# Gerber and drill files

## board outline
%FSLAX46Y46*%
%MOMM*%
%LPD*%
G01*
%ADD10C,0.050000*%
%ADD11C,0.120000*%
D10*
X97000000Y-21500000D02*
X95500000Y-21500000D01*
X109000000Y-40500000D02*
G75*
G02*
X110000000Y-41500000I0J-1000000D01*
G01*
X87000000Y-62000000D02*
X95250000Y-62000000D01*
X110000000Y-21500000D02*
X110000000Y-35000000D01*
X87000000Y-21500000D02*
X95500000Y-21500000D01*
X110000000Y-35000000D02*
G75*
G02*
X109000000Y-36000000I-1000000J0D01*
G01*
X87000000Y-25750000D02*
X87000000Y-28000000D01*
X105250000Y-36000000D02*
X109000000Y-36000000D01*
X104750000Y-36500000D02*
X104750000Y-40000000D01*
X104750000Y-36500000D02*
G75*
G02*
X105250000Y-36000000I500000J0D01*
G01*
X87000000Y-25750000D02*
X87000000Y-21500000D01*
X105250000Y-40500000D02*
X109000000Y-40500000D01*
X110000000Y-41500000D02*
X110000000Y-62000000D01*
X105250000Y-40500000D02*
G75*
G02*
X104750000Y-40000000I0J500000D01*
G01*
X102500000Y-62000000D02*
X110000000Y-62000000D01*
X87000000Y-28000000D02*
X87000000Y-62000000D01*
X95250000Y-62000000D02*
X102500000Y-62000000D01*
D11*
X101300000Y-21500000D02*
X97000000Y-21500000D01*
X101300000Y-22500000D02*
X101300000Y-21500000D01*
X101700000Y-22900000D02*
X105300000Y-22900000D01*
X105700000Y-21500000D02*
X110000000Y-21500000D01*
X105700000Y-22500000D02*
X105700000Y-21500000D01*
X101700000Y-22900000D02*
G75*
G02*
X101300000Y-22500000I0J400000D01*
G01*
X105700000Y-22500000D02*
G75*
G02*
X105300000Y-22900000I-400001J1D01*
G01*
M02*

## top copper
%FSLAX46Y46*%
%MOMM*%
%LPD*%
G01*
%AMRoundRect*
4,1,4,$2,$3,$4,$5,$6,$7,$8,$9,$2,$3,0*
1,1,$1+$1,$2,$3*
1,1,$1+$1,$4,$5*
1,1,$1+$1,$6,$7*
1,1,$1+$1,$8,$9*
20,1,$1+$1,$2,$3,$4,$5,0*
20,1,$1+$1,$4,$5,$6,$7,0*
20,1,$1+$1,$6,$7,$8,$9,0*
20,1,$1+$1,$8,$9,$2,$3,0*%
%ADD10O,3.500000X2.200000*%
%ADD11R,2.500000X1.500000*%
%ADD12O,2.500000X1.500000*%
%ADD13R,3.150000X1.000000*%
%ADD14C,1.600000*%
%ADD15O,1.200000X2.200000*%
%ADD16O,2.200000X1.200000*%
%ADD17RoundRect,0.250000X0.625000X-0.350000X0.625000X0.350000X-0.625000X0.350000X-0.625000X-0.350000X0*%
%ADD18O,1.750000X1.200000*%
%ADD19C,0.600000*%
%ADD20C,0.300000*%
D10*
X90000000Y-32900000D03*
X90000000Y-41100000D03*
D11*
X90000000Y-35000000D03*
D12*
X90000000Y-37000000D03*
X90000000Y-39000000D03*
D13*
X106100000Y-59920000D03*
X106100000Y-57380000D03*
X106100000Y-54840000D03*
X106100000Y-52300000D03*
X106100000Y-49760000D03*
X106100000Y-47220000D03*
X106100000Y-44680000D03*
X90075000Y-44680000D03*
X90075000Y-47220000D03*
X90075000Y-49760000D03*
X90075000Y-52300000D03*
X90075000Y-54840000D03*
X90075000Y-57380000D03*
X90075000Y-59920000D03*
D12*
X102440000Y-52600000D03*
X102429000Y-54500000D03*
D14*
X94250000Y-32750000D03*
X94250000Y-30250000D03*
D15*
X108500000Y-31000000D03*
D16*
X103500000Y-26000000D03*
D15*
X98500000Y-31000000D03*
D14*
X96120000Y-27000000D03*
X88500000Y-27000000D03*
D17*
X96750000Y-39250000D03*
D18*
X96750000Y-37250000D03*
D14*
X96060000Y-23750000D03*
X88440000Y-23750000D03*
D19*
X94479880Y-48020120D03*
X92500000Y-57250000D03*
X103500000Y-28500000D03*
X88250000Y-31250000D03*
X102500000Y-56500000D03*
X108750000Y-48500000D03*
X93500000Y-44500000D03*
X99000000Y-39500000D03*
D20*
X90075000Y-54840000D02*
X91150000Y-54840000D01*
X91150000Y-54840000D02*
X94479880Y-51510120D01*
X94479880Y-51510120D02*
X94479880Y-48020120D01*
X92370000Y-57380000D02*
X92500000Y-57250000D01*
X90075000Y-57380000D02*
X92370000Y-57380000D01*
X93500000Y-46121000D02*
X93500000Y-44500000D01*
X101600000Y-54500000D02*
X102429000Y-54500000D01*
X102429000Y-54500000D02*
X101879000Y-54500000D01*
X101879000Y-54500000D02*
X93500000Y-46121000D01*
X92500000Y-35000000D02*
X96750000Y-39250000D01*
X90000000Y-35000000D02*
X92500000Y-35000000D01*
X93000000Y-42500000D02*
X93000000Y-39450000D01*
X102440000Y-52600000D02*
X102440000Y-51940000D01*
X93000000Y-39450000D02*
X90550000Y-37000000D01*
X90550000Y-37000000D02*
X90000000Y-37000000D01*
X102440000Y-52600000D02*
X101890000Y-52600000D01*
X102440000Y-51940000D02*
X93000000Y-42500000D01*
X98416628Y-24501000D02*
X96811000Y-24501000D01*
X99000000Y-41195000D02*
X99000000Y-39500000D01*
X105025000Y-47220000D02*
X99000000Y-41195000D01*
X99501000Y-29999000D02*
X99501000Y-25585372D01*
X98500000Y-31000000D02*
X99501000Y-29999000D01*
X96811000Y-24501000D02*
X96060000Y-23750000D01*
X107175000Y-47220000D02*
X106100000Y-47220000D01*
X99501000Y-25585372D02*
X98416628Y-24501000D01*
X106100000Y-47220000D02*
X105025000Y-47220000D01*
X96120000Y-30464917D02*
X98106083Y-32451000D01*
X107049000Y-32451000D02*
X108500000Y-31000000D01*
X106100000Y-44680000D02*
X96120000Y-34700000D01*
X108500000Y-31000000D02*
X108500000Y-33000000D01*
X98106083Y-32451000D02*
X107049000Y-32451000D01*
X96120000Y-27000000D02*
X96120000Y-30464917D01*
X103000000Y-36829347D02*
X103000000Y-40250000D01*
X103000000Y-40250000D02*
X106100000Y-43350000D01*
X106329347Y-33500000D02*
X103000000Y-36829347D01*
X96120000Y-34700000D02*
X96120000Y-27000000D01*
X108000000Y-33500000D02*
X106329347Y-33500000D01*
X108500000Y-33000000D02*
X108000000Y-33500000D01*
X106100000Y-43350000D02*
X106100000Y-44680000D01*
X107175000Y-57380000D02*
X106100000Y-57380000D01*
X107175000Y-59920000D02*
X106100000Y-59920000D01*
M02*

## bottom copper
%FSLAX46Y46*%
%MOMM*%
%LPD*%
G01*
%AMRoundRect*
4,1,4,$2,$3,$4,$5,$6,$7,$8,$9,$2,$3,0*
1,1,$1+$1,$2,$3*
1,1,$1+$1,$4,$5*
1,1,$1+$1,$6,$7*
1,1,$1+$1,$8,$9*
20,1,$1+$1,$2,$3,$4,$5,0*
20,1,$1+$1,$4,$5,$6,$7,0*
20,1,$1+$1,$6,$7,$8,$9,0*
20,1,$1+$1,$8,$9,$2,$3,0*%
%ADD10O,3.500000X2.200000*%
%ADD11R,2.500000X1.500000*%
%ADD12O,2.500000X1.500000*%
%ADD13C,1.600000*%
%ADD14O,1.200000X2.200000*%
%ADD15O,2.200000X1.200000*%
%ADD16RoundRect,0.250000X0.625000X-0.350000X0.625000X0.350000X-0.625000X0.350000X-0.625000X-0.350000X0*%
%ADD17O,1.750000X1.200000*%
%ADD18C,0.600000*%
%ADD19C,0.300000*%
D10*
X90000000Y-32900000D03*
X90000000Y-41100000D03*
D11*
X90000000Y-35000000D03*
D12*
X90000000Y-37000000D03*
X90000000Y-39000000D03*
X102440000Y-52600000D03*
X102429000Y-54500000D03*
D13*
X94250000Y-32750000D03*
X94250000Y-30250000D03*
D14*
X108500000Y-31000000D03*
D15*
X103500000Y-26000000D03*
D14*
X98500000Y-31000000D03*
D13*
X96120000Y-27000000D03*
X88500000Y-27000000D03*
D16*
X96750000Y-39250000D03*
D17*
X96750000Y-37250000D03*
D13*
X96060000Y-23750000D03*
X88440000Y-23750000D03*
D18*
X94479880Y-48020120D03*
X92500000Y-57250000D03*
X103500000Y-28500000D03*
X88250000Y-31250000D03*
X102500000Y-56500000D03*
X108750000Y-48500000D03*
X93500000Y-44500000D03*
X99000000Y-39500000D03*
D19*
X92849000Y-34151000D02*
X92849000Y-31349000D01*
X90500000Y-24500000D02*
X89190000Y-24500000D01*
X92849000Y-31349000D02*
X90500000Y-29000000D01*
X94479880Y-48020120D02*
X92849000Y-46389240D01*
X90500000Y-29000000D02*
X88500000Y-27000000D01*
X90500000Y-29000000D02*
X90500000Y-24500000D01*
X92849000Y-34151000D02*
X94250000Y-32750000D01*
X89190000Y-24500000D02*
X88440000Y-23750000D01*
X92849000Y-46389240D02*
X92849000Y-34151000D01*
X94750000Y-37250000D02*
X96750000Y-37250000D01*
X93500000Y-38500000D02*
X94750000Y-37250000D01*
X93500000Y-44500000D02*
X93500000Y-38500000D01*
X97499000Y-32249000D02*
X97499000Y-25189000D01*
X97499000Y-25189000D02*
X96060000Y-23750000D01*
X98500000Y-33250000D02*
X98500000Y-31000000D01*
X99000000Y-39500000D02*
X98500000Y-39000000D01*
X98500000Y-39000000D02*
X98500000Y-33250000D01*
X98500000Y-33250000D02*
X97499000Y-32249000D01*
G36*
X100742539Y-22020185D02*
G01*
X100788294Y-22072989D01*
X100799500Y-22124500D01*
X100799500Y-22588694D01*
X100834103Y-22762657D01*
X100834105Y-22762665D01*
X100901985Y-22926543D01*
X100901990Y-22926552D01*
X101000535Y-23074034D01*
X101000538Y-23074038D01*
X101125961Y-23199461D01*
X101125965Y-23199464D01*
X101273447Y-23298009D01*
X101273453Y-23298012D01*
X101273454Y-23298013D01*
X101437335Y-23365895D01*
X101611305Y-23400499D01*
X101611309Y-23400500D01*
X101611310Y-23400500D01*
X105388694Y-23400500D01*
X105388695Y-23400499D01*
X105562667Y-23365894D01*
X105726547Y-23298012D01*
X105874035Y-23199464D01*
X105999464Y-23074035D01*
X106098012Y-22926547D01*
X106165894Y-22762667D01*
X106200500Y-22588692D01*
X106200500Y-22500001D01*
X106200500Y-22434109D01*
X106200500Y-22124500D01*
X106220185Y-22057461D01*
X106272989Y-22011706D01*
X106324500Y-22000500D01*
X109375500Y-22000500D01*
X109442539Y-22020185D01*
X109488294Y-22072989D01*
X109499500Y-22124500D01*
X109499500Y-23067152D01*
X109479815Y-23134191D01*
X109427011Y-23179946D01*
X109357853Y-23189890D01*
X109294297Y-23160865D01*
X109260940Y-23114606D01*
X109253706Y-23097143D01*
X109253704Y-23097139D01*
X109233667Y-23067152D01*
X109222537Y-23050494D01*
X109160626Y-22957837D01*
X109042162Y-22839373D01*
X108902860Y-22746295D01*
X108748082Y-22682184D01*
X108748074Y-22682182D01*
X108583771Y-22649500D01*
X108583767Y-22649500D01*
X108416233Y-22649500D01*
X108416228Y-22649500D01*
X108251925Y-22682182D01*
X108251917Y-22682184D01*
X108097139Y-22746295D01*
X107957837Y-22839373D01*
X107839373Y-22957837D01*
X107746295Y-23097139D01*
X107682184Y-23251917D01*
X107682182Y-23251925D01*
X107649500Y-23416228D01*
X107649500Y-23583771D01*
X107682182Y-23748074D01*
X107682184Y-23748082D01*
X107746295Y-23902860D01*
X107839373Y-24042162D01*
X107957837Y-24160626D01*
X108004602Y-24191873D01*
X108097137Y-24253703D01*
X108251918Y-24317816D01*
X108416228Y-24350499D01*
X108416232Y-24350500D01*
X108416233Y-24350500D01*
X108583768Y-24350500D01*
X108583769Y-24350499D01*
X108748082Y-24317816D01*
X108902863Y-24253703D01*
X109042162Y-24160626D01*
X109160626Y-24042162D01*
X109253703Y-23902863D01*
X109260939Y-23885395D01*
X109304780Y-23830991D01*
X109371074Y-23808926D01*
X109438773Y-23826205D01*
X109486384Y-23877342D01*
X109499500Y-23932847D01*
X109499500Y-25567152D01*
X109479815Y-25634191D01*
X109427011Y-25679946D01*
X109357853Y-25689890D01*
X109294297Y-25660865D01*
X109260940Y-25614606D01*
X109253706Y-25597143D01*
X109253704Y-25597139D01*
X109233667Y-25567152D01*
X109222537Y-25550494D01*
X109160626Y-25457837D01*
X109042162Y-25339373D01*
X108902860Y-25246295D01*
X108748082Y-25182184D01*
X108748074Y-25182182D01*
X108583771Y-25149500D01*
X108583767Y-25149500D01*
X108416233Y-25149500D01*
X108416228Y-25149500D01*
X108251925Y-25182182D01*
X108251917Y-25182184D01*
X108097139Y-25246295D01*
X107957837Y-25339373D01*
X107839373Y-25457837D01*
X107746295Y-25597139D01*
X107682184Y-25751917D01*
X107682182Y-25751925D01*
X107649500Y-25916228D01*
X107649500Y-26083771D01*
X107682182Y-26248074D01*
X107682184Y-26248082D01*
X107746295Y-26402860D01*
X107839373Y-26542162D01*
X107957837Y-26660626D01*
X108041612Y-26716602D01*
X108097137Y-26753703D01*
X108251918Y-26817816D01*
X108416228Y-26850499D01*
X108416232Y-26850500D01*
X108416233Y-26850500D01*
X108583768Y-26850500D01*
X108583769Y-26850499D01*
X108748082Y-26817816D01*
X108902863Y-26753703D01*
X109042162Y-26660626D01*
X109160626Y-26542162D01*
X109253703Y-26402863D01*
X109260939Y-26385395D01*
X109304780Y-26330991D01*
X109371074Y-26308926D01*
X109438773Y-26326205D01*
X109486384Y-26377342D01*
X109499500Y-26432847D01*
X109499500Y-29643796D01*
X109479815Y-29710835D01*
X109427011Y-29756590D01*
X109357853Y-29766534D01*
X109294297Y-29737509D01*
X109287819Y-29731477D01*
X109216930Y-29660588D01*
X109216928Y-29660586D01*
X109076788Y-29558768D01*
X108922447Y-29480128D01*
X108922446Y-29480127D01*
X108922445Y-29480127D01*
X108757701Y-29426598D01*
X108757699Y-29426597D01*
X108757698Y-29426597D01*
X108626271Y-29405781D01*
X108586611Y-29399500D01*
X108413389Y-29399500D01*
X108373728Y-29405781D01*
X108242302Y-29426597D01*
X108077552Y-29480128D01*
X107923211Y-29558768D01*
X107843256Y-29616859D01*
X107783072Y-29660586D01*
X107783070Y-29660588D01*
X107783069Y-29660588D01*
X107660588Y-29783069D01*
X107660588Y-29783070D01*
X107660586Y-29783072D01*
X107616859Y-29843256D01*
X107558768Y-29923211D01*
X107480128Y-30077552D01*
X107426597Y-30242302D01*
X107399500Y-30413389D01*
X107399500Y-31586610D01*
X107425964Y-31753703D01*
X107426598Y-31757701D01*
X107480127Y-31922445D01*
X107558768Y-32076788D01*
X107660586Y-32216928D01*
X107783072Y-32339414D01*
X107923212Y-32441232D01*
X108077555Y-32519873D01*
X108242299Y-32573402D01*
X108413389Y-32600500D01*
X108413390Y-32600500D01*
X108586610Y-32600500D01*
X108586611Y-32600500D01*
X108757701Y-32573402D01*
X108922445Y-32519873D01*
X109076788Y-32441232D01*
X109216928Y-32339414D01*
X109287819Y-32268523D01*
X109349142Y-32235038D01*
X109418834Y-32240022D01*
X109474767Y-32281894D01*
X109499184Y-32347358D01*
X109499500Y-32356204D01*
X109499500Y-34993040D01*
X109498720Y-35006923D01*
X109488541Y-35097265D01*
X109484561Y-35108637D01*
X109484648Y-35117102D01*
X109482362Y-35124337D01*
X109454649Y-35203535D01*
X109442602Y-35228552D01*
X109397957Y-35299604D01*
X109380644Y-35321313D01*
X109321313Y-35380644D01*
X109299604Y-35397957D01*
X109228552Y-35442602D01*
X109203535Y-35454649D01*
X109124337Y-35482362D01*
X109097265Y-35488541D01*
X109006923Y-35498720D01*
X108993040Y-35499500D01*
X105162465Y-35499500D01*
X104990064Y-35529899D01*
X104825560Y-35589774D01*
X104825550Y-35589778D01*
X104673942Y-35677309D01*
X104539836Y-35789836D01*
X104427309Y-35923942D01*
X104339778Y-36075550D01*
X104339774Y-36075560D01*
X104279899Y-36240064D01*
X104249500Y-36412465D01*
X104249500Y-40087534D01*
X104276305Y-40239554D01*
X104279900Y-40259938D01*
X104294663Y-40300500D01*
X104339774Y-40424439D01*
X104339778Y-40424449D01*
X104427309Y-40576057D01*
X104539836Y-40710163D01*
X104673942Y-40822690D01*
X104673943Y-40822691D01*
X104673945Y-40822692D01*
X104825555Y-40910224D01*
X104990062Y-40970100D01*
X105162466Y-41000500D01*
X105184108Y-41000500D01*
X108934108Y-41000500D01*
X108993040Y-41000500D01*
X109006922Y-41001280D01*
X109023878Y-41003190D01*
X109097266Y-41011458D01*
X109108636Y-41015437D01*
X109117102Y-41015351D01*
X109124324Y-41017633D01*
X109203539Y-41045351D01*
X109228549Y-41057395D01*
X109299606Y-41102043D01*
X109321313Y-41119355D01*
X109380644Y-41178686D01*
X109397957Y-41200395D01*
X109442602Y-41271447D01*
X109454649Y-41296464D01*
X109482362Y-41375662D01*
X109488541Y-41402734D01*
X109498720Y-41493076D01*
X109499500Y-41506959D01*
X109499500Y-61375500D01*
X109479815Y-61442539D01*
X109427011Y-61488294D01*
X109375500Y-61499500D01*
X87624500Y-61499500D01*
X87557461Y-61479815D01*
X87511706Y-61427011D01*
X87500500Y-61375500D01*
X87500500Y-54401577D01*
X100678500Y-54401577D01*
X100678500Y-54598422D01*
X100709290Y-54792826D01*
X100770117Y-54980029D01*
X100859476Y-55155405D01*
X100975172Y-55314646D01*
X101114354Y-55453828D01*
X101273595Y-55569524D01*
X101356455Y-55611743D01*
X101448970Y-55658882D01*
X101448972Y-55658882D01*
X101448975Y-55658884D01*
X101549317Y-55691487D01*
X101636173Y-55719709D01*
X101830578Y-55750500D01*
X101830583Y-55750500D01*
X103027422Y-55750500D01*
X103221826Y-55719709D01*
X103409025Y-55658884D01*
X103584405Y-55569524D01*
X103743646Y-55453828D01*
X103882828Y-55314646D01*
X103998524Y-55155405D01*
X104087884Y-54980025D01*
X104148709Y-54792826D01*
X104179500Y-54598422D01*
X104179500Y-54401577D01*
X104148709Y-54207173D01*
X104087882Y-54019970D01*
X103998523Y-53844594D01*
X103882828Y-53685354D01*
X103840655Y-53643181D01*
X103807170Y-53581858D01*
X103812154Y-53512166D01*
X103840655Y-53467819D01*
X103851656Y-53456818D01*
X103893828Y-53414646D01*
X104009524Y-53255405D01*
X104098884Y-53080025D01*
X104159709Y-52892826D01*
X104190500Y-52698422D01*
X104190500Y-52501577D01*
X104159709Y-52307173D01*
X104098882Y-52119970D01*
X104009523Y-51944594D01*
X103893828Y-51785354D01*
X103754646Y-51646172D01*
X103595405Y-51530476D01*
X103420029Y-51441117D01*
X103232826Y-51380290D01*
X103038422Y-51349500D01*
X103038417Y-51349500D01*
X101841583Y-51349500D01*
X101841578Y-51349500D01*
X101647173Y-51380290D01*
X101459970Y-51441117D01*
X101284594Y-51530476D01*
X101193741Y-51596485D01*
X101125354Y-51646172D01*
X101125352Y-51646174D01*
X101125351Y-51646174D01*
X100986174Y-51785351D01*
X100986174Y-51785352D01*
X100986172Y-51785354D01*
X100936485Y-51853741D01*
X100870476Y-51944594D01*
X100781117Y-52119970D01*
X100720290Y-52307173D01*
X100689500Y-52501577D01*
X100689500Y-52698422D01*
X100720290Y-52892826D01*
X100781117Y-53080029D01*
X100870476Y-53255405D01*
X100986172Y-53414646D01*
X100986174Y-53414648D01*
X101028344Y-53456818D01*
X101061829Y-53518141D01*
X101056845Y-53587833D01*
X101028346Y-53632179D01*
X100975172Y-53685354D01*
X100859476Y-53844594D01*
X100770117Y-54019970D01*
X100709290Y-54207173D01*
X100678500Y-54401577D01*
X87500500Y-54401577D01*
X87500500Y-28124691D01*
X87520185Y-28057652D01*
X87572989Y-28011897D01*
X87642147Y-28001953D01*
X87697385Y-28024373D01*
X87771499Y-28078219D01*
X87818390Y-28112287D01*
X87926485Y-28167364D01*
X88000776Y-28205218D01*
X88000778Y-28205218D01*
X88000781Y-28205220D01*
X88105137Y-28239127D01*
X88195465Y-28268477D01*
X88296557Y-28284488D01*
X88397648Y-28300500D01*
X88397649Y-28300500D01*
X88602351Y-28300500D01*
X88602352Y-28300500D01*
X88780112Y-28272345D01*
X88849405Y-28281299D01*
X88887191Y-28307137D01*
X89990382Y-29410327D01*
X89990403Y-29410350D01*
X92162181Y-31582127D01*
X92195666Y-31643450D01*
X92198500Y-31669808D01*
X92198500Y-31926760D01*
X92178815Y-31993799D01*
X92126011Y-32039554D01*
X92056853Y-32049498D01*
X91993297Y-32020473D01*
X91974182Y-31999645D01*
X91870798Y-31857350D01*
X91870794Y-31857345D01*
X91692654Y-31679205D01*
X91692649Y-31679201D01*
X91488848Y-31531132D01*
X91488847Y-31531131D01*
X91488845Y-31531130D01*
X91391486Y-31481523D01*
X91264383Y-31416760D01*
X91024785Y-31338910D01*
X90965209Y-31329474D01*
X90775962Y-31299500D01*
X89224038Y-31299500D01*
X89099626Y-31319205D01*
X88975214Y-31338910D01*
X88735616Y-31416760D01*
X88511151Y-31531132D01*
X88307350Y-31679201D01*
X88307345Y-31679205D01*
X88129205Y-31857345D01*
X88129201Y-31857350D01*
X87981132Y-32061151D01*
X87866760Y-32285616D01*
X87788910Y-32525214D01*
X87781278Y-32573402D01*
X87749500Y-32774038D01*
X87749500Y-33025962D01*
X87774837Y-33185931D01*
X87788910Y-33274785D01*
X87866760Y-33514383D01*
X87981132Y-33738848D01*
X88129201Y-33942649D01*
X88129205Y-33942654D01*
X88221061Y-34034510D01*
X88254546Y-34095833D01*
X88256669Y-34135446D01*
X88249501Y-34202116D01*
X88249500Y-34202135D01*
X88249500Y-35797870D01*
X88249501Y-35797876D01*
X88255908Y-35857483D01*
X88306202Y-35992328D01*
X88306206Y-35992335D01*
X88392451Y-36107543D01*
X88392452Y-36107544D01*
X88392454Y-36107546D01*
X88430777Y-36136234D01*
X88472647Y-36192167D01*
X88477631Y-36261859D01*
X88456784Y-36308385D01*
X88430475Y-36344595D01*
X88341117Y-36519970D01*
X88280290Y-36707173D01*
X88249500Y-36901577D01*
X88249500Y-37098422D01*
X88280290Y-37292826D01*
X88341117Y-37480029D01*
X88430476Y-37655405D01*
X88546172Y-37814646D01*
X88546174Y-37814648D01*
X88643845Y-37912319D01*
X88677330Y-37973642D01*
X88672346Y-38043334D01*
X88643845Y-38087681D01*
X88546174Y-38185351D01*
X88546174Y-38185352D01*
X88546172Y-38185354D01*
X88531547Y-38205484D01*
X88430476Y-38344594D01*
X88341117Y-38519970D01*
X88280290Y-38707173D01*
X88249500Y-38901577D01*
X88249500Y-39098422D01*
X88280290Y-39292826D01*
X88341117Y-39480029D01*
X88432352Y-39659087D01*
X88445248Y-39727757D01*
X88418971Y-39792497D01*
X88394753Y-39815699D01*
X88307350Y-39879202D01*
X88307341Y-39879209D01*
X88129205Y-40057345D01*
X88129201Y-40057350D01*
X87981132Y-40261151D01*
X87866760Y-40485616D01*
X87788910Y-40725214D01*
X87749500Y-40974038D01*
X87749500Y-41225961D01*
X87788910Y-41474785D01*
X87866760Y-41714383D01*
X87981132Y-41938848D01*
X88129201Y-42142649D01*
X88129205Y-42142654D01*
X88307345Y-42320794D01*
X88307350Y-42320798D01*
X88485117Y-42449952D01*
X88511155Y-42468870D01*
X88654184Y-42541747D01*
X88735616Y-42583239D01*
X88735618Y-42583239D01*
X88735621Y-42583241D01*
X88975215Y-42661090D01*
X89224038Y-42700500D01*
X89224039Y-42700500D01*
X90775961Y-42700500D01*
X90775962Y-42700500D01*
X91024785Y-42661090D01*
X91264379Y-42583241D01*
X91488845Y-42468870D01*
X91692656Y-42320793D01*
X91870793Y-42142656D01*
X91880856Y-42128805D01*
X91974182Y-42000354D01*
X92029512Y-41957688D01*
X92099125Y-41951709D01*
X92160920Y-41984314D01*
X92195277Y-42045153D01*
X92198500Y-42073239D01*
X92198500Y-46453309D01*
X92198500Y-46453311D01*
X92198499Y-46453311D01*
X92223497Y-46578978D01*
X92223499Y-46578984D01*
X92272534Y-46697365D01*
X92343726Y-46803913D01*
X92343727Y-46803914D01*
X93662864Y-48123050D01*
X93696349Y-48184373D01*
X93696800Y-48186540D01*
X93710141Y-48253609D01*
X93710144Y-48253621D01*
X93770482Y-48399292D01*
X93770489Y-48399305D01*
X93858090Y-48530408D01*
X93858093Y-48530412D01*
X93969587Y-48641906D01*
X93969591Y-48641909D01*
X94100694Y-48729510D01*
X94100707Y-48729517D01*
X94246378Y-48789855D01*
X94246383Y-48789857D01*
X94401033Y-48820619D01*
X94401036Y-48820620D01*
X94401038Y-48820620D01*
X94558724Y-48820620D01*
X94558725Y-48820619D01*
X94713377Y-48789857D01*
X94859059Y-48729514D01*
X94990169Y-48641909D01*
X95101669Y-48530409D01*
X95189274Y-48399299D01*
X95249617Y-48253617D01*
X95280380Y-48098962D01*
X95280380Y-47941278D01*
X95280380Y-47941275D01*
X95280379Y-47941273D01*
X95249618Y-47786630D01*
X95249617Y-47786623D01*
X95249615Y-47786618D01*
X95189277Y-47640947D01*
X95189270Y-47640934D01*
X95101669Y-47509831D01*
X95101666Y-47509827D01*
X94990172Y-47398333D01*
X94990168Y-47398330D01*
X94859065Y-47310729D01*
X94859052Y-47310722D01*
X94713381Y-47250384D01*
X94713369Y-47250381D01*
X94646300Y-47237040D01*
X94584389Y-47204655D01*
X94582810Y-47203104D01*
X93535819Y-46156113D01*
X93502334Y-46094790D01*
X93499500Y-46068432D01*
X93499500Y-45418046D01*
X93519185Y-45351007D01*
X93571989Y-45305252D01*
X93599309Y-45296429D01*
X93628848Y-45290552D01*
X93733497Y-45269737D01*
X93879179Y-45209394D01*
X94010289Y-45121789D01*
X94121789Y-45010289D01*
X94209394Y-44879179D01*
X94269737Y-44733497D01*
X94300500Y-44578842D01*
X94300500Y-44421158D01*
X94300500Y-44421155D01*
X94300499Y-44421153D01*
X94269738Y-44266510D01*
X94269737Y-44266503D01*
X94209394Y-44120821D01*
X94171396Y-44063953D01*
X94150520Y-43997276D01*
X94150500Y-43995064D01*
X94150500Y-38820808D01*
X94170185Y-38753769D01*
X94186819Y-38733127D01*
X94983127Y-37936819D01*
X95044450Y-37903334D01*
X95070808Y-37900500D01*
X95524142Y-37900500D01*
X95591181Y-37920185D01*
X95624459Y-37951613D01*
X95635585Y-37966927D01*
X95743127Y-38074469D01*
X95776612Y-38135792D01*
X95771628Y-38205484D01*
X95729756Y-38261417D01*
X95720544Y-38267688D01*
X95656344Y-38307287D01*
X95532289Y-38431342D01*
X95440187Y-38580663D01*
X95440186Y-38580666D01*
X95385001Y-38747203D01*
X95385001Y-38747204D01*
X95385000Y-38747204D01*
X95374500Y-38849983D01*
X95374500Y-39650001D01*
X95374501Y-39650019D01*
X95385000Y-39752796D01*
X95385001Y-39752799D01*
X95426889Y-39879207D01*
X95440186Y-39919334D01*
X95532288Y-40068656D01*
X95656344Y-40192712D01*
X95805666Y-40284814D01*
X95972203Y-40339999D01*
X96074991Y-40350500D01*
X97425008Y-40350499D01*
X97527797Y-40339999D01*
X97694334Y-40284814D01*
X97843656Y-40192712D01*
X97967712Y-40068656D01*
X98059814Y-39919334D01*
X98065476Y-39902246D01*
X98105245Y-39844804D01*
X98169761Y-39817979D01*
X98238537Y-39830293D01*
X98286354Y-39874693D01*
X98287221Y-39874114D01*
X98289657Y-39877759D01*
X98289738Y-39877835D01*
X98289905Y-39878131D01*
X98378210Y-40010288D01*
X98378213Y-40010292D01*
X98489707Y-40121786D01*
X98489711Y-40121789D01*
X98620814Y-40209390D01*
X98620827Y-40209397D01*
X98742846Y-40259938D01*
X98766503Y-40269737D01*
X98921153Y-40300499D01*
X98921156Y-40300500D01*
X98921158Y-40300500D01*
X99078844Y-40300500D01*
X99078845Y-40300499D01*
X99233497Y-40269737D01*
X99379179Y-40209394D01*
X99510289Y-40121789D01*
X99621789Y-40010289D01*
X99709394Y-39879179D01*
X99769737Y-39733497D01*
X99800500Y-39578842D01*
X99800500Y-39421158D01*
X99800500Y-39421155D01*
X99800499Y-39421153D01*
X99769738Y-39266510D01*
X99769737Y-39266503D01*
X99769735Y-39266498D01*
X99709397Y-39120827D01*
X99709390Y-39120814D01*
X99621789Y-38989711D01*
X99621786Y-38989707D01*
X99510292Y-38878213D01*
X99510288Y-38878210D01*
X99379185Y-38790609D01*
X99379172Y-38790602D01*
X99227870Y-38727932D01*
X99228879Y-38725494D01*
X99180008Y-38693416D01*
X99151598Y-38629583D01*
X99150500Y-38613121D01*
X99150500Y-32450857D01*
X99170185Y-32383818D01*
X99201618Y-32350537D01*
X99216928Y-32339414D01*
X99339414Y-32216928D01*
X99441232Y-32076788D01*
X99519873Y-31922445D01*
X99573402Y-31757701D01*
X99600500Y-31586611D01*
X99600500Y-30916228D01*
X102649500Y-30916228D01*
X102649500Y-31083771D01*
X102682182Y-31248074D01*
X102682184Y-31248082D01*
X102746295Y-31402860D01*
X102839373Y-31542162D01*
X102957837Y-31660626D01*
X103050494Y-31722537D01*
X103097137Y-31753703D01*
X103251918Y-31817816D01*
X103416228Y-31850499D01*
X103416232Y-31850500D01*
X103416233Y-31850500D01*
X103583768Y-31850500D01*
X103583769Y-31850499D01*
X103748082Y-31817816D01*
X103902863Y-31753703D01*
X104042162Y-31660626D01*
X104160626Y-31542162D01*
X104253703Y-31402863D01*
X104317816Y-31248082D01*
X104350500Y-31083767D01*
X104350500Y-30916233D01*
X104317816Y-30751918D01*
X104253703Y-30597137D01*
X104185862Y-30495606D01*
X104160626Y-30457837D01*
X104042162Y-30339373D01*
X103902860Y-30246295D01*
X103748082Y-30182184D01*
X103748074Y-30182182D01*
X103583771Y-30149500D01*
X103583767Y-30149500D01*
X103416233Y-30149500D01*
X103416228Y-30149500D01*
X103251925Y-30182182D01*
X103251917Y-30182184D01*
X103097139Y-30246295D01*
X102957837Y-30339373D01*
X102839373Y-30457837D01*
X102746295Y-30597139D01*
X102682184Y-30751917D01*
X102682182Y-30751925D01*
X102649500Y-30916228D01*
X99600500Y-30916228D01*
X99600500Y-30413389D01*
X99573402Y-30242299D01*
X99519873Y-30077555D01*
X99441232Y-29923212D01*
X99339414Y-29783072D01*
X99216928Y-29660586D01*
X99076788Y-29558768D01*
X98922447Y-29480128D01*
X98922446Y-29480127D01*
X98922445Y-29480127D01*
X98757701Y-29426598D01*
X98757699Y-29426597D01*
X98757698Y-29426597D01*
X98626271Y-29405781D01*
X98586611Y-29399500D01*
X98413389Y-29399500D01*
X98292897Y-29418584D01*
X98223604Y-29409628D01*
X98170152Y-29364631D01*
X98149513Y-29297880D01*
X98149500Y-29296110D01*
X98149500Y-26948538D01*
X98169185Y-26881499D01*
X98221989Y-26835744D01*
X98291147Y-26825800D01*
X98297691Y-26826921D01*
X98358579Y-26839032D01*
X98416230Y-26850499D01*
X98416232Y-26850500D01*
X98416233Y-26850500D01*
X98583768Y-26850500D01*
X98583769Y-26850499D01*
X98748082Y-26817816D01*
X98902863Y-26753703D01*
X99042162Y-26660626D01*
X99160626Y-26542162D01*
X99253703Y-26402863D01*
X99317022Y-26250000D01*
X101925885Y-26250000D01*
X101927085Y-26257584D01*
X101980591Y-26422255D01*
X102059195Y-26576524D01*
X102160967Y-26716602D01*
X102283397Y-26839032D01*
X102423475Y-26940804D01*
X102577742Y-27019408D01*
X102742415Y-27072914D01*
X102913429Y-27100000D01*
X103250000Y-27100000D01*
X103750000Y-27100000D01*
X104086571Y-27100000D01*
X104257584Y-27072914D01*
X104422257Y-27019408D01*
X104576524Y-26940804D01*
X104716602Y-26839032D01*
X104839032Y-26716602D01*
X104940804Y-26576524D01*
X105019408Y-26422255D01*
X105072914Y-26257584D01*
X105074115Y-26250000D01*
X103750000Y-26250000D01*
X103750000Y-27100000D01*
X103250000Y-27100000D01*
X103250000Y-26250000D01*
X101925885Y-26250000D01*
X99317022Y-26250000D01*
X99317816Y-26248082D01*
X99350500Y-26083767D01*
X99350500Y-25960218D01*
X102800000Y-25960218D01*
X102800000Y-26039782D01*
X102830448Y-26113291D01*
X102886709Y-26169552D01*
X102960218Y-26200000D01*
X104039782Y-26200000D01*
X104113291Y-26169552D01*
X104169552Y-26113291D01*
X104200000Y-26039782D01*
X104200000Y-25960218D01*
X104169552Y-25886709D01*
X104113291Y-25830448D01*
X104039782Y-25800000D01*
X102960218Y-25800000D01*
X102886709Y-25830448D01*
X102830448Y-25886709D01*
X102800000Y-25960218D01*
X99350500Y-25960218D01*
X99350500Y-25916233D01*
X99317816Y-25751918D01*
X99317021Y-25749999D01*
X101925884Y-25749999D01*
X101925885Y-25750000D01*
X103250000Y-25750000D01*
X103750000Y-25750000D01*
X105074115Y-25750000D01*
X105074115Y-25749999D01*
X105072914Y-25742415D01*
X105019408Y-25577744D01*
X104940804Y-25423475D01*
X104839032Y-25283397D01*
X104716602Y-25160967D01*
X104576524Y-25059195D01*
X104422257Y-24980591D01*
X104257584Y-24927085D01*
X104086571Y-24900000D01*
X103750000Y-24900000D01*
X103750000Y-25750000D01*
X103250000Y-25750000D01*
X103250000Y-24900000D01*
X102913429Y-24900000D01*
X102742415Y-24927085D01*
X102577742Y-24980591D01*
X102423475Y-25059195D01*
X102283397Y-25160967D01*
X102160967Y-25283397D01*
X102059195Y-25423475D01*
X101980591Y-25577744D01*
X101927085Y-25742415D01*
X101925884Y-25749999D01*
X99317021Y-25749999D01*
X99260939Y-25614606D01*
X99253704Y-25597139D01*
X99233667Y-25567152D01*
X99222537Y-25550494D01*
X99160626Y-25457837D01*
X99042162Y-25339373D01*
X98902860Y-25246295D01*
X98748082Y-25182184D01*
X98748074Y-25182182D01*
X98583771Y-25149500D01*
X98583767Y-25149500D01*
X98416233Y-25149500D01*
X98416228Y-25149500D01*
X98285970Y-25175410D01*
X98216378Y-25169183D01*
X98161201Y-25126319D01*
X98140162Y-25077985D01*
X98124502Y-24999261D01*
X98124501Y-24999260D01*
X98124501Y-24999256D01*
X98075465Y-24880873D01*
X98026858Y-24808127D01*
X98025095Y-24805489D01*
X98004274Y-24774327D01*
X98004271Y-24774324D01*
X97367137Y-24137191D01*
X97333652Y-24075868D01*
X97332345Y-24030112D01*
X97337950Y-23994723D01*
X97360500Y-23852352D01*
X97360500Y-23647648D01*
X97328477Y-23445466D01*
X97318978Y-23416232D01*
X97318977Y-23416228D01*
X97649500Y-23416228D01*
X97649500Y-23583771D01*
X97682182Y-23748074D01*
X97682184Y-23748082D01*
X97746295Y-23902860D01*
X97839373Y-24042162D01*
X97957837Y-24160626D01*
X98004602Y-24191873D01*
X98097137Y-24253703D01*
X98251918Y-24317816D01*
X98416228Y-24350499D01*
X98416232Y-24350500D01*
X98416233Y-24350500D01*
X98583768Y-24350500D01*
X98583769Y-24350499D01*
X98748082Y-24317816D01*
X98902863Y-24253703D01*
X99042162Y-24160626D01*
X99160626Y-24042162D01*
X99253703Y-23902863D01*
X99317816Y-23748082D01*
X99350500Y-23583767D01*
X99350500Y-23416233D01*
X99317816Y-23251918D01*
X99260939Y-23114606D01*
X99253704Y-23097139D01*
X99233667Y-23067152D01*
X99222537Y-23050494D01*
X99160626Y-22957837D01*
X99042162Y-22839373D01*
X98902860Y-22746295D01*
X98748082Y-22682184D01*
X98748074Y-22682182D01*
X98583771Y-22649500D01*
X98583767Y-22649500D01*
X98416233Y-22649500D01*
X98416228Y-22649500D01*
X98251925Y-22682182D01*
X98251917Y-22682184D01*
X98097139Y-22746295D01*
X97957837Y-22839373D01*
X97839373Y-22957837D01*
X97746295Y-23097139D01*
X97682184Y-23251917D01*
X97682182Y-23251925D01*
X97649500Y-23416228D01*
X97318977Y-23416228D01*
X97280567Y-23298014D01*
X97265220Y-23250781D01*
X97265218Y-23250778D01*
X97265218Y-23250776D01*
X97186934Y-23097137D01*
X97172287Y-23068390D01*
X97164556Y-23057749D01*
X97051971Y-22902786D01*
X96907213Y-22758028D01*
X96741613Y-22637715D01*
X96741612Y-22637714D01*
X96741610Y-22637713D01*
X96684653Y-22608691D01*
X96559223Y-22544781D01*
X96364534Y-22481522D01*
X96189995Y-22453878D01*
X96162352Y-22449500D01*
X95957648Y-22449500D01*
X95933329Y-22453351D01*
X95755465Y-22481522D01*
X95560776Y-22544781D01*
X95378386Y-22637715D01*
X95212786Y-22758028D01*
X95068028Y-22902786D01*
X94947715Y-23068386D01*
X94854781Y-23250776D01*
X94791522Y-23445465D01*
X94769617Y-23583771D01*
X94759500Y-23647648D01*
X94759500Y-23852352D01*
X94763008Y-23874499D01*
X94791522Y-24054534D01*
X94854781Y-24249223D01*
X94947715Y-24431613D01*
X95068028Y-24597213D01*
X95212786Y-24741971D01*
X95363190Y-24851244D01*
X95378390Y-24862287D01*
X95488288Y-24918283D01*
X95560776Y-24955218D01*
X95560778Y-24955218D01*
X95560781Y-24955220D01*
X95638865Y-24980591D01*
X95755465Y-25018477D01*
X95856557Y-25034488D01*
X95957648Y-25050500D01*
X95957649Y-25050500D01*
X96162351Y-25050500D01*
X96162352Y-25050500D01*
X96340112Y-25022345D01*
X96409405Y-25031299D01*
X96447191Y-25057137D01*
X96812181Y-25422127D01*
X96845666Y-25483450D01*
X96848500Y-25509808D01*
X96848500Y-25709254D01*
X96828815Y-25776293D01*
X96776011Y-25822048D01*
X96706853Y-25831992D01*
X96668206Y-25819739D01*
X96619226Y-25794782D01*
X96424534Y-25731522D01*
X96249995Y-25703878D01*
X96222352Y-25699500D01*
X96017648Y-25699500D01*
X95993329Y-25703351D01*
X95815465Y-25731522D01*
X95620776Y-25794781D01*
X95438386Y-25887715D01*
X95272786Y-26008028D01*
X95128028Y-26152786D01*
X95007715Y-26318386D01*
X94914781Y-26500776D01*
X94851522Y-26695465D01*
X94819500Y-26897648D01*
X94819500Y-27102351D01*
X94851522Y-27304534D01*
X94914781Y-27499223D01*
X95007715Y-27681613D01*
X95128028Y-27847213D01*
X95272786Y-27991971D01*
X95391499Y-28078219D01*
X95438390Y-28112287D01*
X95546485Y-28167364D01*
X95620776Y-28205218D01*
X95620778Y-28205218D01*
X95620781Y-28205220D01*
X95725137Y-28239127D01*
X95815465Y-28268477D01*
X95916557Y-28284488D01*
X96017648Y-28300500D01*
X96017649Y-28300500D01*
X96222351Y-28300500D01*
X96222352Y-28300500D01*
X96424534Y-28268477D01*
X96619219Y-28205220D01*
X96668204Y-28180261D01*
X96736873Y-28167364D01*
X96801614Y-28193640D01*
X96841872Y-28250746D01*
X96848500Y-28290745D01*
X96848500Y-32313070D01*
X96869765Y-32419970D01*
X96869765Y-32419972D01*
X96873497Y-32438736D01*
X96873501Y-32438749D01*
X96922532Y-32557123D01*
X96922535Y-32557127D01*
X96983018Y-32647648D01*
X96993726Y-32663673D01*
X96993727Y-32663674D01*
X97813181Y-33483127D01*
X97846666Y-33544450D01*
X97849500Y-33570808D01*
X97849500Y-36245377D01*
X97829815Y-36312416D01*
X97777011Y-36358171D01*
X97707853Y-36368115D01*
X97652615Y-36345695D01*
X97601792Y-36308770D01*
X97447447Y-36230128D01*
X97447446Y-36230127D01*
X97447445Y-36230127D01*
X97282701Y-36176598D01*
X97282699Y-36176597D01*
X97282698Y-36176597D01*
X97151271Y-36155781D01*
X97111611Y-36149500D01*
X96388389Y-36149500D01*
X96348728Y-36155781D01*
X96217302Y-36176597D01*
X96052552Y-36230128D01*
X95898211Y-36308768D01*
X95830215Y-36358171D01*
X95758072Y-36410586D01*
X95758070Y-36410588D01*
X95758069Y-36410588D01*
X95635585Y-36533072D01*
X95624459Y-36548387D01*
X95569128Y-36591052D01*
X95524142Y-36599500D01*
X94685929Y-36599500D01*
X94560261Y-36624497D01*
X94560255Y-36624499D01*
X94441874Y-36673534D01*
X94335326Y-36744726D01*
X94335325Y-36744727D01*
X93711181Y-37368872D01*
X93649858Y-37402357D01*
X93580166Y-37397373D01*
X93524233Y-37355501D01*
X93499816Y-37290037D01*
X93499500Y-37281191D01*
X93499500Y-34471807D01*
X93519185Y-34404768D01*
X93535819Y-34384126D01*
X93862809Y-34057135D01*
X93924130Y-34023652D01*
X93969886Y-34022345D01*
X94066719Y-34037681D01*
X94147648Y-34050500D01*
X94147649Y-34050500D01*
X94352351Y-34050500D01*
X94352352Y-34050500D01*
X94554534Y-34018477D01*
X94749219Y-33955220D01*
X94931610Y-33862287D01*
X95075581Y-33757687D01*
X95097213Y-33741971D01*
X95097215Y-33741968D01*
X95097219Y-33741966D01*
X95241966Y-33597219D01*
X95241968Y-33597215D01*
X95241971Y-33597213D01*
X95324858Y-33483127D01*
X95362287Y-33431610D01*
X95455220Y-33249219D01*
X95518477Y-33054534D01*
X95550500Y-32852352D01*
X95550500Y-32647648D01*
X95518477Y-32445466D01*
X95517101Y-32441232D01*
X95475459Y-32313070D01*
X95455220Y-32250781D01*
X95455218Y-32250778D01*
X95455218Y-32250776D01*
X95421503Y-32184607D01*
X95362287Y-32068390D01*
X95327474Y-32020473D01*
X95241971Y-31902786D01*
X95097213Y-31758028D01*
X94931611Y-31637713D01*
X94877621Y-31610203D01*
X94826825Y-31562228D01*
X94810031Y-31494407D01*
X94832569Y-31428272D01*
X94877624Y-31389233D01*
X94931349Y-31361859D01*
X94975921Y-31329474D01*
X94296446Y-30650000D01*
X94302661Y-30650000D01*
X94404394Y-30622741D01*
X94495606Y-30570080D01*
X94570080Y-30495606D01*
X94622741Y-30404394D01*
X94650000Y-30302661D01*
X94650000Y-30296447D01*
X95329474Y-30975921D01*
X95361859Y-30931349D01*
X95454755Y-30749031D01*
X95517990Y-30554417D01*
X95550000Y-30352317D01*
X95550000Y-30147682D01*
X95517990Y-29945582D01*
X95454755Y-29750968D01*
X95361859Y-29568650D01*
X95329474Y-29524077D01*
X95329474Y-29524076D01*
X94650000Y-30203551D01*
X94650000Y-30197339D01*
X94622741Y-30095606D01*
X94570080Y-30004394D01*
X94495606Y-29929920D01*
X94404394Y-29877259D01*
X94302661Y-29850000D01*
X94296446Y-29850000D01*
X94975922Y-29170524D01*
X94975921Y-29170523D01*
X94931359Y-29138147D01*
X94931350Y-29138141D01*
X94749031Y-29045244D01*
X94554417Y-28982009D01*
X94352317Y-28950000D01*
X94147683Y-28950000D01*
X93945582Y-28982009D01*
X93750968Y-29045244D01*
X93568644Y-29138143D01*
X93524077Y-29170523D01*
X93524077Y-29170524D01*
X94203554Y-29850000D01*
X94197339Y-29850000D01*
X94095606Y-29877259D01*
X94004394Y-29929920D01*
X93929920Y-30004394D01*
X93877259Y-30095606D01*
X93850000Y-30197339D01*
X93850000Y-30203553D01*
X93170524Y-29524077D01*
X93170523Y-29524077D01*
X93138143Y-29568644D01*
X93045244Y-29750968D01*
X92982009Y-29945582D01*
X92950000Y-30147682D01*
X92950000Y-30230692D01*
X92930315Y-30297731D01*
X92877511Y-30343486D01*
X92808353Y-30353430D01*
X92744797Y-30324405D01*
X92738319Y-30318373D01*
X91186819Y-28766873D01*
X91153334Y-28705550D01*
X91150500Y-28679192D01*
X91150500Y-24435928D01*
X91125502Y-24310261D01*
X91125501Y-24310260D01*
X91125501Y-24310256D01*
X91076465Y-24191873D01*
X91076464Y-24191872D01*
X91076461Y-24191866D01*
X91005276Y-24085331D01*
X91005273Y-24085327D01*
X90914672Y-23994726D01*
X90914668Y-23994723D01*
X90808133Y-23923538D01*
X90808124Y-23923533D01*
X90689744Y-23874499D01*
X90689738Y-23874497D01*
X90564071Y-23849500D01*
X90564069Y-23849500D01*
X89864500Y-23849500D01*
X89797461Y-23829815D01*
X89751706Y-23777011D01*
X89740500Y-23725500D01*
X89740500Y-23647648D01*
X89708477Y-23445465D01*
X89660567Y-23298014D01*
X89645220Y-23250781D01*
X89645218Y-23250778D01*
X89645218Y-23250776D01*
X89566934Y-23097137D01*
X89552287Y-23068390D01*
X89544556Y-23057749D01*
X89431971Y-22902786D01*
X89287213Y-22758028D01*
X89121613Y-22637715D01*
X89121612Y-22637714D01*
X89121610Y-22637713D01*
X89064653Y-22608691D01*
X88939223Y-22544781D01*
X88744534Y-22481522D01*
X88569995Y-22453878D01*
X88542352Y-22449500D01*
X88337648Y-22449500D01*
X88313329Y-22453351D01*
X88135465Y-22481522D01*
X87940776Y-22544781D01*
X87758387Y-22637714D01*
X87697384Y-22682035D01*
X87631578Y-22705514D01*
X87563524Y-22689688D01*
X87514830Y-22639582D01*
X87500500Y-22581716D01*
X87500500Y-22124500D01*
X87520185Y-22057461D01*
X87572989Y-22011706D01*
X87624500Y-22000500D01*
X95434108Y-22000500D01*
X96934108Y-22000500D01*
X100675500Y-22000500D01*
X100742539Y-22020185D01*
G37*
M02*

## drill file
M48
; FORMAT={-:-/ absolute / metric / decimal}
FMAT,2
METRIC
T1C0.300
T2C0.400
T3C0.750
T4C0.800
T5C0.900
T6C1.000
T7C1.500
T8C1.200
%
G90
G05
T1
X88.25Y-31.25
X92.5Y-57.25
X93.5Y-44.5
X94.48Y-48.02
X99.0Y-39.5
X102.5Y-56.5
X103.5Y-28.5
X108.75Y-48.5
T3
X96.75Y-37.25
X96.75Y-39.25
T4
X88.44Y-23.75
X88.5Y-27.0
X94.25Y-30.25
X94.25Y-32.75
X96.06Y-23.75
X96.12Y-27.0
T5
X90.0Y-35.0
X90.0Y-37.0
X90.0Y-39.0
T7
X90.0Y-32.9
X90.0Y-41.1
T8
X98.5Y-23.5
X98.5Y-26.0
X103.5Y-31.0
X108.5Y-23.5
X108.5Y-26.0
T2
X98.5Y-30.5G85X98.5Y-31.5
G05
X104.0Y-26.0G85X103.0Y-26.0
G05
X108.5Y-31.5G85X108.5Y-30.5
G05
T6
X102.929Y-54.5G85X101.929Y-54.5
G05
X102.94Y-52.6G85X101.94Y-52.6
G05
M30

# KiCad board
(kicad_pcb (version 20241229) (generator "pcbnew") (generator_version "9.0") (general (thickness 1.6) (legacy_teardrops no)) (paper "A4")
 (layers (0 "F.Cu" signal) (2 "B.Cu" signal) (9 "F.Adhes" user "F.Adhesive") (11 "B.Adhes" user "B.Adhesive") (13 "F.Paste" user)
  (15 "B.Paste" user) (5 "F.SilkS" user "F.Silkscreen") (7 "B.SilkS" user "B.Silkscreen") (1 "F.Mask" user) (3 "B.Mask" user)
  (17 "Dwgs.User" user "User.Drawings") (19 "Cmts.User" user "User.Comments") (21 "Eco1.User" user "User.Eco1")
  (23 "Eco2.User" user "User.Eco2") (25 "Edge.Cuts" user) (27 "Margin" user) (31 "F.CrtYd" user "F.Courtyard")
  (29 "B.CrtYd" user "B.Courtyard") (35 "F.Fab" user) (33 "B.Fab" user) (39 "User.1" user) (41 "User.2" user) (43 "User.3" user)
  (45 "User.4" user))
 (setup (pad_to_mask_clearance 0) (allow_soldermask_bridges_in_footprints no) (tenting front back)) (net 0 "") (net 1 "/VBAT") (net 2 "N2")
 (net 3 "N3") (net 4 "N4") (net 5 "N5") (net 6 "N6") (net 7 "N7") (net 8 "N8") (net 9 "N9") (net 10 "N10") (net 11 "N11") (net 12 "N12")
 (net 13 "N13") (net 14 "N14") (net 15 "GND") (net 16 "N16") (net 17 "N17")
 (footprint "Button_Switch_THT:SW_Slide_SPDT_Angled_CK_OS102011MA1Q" (layer "F.Cu") (at 90 35 -90)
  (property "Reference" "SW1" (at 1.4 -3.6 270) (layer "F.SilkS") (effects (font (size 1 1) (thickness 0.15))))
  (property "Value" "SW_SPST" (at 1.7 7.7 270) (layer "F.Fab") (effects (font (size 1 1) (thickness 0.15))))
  (pad "" thru_hole oval (at -2.1 0 270) (size 2.2 3.5) (drill 1.5) (layers "*.Cu" "*.Mask") (remove_unused_layers no))
  (pad "" thru_hole oval (at 6.1 0 270) (size 2.2 3.5) (drill 1.5) (layers "*.Cu" "*.Mask") (remove_unused_layers no))
  (pad "1" thru_hole rect (at 0 0 270) (size 1.5 2.5) (drill 0.9) (layers "*.Cu" "*.Mask") (remove_unused_layers no) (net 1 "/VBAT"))
  (pad "2" thru_hole oval (at 2 0 270) (size 1.5 2.5) (drill 0.9) (layers "*.Cu" "*.Mask") (remove_unused_layers no) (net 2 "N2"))
  (pad "3" thru_hole oval (at 4 0 270) (size 1.5 2.5) (drill 0.9) (layers "*.Cu" "*.Mask") (remove_unused_layers no)))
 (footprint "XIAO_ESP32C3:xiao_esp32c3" (layer "F.Cu") (at 97.5 50.5 180)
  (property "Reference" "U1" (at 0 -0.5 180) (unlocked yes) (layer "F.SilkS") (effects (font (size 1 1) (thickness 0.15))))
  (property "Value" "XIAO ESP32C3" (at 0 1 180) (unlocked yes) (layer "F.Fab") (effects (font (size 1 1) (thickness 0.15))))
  (pad "1" smd rect (at -8.6 -9.42 180) (size 3.15 1) (layers "F.Cu" "F.Mask" "F.Paste") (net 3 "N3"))
  (pad "2" smd rect (at -8.6 -6.88 180) (size 3.15 1) (layers "F.Cu" "F.Mask" "F.Paste") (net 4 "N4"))
  (pad "3" smd rect (at -8.6 -4.34 180) (size 3.15 1) (layers "F.Cu" "F.Mask" "F.Paste") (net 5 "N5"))
  (pad "4" smd rect (at -8.6 -1.8 180) (size 3.15 1) (layers "F.Cu" "F.Mask" "F.Paste") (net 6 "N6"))
  (pad "5" smd rect (at -8.6 0.74 180) (size 3.15 1) (layers "F.Cu" "F.Mask" "F.Paste") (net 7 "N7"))
  (pad "6" smd rect (at -8.6 3.28 180) (size 3.15 1) (layers "F.Cu" "F.Mask" "F.Paste") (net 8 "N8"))
  (pad "7" smd rect (at -8.6 5.82 180) (size 3.15 1) (layers "F.Cu" "F.Mask" "F.Paste") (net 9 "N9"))
  (pad "8" smd rect (at 7.425 5.82 180) (size 3.15 1) (layers "F.Cu" "F.Mask" "F.Paste") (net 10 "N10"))
  (pad "9" smd rect (at 7.425 3.28 180) (size 3.15 1) (layers "F.Cu" "F.Mask" "F.Paste") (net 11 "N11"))
  (pad "10" smd rect (at 7.425 0.74 180) (size 3.15 1) (layers "F.Cu" "F.Mask" "F.Paste") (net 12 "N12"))
  (pad "11" smd rect (at 7.425 -1.8 180) (size 3.15 1) (layers "F.Cu" "F.Mask" "F.Paste") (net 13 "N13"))
  (pad "12" smd rect (at 7.425 -4.34 180) (size 3.15 1) (layers "F.Cu" "F.Mask" "F.Paste") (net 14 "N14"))
  (pad "13" smd rect (at 7.425 -6.88 180) (size 3.15 1) (layers "F.Cu" "F.Mask" "F.Paste") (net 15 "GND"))
  (pad "14" smd rect (at 7.425 -9.42 180) (size 3.15 1) (layers "F.Cu" "F.Mask" "F.Paste") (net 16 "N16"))
  (pad "B+" thru_hole oval (at -4.94 -2.1 180) (size 2.5 1.5) (drill oval 2 1) (layers "*.Cu" "*.Mask") (remove_unused_layers no)
   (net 2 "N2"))
  (pad "B-" thru_hole oval (at -4.929 -4 180) (size 2.5 1.5) (drill oval 2 1) (layers "*.Cu" "*.Mask") (remove_unused_layers no)
   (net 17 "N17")))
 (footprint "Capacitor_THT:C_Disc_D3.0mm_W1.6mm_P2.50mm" (layer "F.Cu") (at 94.25 32.75 90)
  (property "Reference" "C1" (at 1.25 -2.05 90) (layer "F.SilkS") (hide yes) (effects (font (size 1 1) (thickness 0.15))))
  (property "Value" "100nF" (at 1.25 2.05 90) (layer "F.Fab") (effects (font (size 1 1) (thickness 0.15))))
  (pad "1" thru_hole circle (at 0 0 90) (size 1.6 1.6) (drill 0.8) (layers "*.Cu" "*.Mask") (remove_unused_layers no) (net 14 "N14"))
  (pad "2" thru_hole circle (at 2.5 0 90) (size 1.6 1.6) (drill 0.8) (layers "*.Cu" "*.Mask") (remove_unused_layers no) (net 15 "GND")))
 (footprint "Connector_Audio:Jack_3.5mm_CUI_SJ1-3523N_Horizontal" (layer "F.Cu") (at 103.5 26 180)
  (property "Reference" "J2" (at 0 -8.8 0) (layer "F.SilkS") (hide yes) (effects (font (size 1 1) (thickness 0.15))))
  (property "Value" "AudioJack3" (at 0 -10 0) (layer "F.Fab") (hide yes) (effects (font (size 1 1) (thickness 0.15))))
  (fp_line (start 2.2 4.5) (end 6.5 4.5) (stroke (width 0.12) (type solid)) (layer "Edge.Cuts"))
  (fp_line (start 2.2 3.5) (end 2.2 4.5) (stroke (width 0.12) (type solid)) (layer "Edge.Cuts"))
  (fp_line (start 1.8 3.1) (end -1.8 3.1) (stroke (width 0.12) (type solid)) (layer "Edge.Cuts"))
  (fp_line (start -2.2 4.5) (end -6.5 4.5) (stroke (width 0.12) (type solid)) (layer "Edge.Cuts"))
  (fp_line (start -2.2 3.5) (end -2.2 4.5) (stroke (width 0.12) (type solid)) (layer "Edge.Cuts"))
  (fp_arc (start 1.8 3.1) (mid 2.082843 3.217157) (end 2.2 3.5) (stroke (width 0.12) (type solid)) (layer "Edge.Cuts"))
  (fp_arc (start -2.2 3.5) (mid -2.082843 3.217158) (end -1.8 3.1) (stroke (width 0.12) (type solid)) (layer "Edge.Cuts"))
  (pad "" np_thru_hole circle (at -5 0 180) (size 1.2 1.2) (drill 1.2) (layers "*.Cu" "*.Mask"))
  (pad "" np_thru_hole circle (at -5 2.5 180) (size 1.2 1.2) (drill 1.2) (layers "*.Cu" "*.Mask"))
  (pad "" np_thru_hole circle (at 0 -5 180) (size 1.2 1.2) (drill 1.2) (layers "*.Cu" "*.Mask"))
  (pad "" np_thru_hole circle (at 5 0 180) (size 1.2 1.2) (drill 1.2) (layers "*.Cu" "*.Mask"))
  (pad "" np_thru_hole circle (at 5 2.5 180) (size 1.2 1.2) (drill 1.2) (layers "*.Cu" "*.Mask"))
  (pad "R" thru_hole oval (at -5 -5 180) (size 1.2 2.2) (drill oval 0.4 1.4) (layers "*.Cu" "*.Mask") (remove_unused_layers no) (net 9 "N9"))
  (pad "S" thru_hole oval (at 0 0 180) (size 2.2 1.2) (drill oval 1.4 0.4) (layers "*.Cu" "*.Mask") (remove_unused_layers no) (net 15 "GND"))
  (pad "T" thru_hole oval (at 5 -5) (size 1.2 2.2) (drill oval 0.4 1.4) (layers "*.Cu" "*.Mask") (remove_unused_layers no) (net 8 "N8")))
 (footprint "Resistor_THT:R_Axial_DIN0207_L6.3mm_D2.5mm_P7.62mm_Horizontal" (layer "F.Cu") (at 96.12 27 180)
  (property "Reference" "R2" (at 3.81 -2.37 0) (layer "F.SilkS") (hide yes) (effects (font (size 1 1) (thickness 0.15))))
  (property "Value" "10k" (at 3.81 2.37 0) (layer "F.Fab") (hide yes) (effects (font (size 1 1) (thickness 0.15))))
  (pad "1" thru_hole circle (at 0 0 180) (size 1.6 1.6) (drill 0.8) (layers "*.Cu" "*.Mask") (remove_unused_layers no) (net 9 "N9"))
  (pad "2" thru_hole circle (at 7.62 0 180) (size 1.6 1.6) (drill 0.8) (layers "*.Cu" "*.Mask") (remove_unused_layers no) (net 14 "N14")))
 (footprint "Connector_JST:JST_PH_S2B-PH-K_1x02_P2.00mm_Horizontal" (layer "F.Cu") (at 96.75 39.25 90)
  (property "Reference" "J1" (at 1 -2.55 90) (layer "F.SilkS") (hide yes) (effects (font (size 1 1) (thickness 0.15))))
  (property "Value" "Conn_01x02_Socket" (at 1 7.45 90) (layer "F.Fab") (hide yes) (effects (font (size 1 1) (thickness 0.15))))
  (pad "1" thru_hole roundrect (at 0 0 90) (size 1.2 1.75) (drill 0.75) (layers "*.Cu" "*.Mask") (remove_unused_layers no)
   (roundrect_rratio 0.208333) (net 1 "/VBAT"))
  (pad "2" thru_hole oval (at 2 0 90) (size 1.2 1.75) (drill 0.75) (layers "*.Cu" "*.Mask") (remove_unused_layers no) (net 17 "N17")))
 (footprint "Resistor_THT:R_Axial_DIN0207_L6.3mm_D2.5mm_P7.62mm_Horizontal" (layer "F.Cu") (at 96.06 23.75 180)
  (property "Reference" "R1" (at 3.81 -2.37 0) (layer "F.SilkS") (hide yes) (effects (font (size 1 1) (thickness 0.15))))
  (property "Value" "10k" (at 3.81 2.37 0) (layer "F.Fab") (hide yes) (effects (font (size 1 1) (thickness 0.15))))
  (pad "1" thru_hole circle (at 0 0 180) (size 1.6 1.6) (drill 0.8) (layers "*.Cu" "*.Mask") (remove_unused_layers no) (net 8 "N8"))
  (pad "2" thru_hole circle (at 7.62 0 180) (size 1.6 1.6) (drill 0.8) (layers "*.Cu" "*.Mask") (remove_unused_layers no) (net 14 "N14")))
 (gr_line (start 97 21.5) (end 95.5 21.5) (stroke (width 0.05) (type default)) (layer "Edge.Cuts"))
 (gr_arc (start 109 40.5) (mid 109.707107 40.792893) (end 110 41.5) (stroke (width 0.05) (type default)) (layer "Edge.Cuts"))
 (gr_line (start 87 62) (end 95.25 62) (stroke (width 0.05) (type default)) (layer "Edge.Cuts"))
 (gr_line (start 110 21.5) (end 110 35) (stroke (width 0.05) (type default)) (layer "Edge.Cuts"))
 (gr_line (start 87 21.5) (end 95.5 21.5) (stroke (width 0.05) (type default)) (layer "Edge.Cuts"))
 (gr_arc (start 110 35) (mid 109.707107 35.707107) (end 109 36) (stroke (width 0.05) (type default)) (layer "Edge.Cuts"))
 (gr_line (start 87 25.75) (end 87 28) (stroke (width 0.05) (type default)) (layer "Edge.Cuts"))
 (gr_line (start 105.25 36) (end 109 36) (stroke (width 0.05) (type default)) (layer "Edge.Cuts"))
 (gr_line (start 104.75 36.5) (end 104.75 40) (stroke (width 0.05) (type default)) (layer "Edge.Cuts"))
 (gr_arc (start 104.75 36.5) (mid 104.896447 36.146447) (end 105.25 36) (stroke (width 0.05) (type default)) (layer "Edge.Cuts"))
 (gr_line (start 87 25.75) (end 87 21.5) (stroke (width 0.05) (type default)) (layer "Edge.Cuts"))
 (gr_line (start 105.25 40.5) (end 109 40.5) (stroke (width 0.05) (type default)) (layer "Edge.Cuts"))
 (gr_line (start 110 41.5) (end 110 62) (stroke (width 0.05) (type default)) (layer "Edge.Cuts"))
 (gr_arc (start 105.25 40.5) (mid 104.896447 40.353553) (end 104.75 40) (stroke (width 0.05) (type default)) (layer "Edge.Cuts"))
 (gr_line (start 102.5 62) (end 110 62) (stroke (width 0.05) (type default)) (layer "Edge.Cuts"))
 (gr_line (start 87 28) (end 87 62) (stroke (width 0.05) (type default)) (layer "Edge.Cuts"))
 (gr_line (start 95.25 62) (end 102.5 62) (stroke (width 0.05) (type default)) (layer "Edge.Cuts"))
 (segment (start 90.075 54.84) (end 91.15 54.84) (width 0.3) (layer "F.Cu") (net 14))
 (segment (start 91.15 54.84) (end 94.47988 51.51012) (width 0.3) (layer "F.Cu") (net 14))
 (segment (start 94.47988 51.51012) (end 94.47988 48.02012) (width 0.3) (layer "F.Cu") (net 14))
 (via (at 94.47988 48.02012) (size 0.6) (drill 0.3) (layers "F.Cu" "B.Cu") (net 14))
 (segment (start 92.849 34.151) (end 92.849 31.349) (width 0.3) (layer "B.Cu") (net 14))
 (segment (start 90.5 24.5) (end 89.19 24.5) (width 0.3) (layer "B.Cu") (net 14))
 (segment (start 92.849 31.349) (end 90.5 29) (width 0.3) (layer "B.Cu") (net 14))
 (segment (start 94.47988 48.02012) (end 92.849 46.38924) (width 0.3) (layer "B.Cu") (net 14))
 (segment (start 90.5 29) (end 88.5 27) (width 0.3) (layer "B.Cu") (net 14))
 (segment (start 90.5 29) (end 90.5 24.5) (width 0.3) (layer "B.Cu") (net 14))
 (segment (start 92.849 34.151) (end 94.25 32.75) (width 0.3) (layer "B.Cu") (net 14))
 (segment (start 89.19 24.5) (end 88.44 23.75) (width 0.3) (layer "B.Cu") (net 14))
 (segment (start 92.849 46.38924) (end 92.849 34.151) (width 0.3) (layer "B.Cu") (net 14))
 (segment (start 92.37 57.38) (end 92.5 57.25) (width 0.3) (layer "F.Cu") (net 15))
 (segment (start 90.075 57.38) (end 92.37 57.38) (width 0.3) (layer "F.Cu") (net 15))
 (via (at 92.5 57.25) (size 0.6) (drill 0.3) (layers "F.Cu" "B.Cu") (free yes) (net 15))
 (via (at 103.5 28.5) (size 0.6) (drill 0.3) (layers "F.Cu" "B.Cu") (free yes) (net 15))
 (via (at 88.25 31.25) (size 0.6) (drill 0.3) (layers "F.Cu" "B.Cu") (free yes) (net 15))
 (via (at 102.5 56.5) (size 0.6) (drill 0.3) (layers "F.Cu" "B.Cu") (free yes) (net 15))
 (via (at 108.75 48.5) (size 0.6) (drill 0.3) (layers "F.Cu" "B.Cu") (free yes) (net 15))
 (segment (start 93.5 46.121) (end 93.5 44.5) (width 0.3) (layer "F.Cu") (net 17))
 (segment (start 101.6 54.5) (end 102.429 54.5) (width 0.3) (layer "F.Cu") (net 17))
 (segment (start 102.429 54.5) (end 101.879 54.5) (width 0.3) (layer "F.Cu") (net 17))
 (segment (start 101.879 54.5) (end 93.5 46.121) (width 0.3) (layer "F.Cu") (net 17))
 (via (at 93.5 44.5) (size 0.6) (drill 0.3) (layers "F.Cu" "B.Cu") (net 17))
 (segment (start 94.75 37.25) (end 96.75 37.25) (width 0.3) (layer "B.Cu") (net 17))
 (segment (start 93.5 38.5) (end 94.75 37.25) (width 0.3) (layer "B.Cu") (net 17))
 (segment (start 93.5 44.5) (end 93.5 38.5) (width 0.3) (layer "B.Cu") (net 17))
 (segment (start 92.5 35) (end 96.75 39.25) (width 0.3) (layer "F.Cu") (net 1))
 (segment (start 90 35) (end 92.5 35) (width 0.3) (layer "F.Cu") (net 1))
 (segment (start 93 42.5) (end 93 39.45) (width 0.3) (layer "F.Cu") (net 2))
 (segment (start 102.44 52.6) (end 102.44 51.94) (width 0.3) (layer "F.Cu") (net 2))
 (segment (start 93 39.45) (end 90.55 37) (width 0.3) (layer "F.Cu") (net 2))
 (segment (start 90.55 37) (end 90 37) (width 0.3) (layer "F.Cu") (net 2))
 (segment (start 102.44 52.6) (end 101.89 52.6) (width 0.3) (layer "F.Cu") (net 2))
 (segment (start 102.44 51.94) (end 93 42.5) (width 0.3) (layer "F.Cu") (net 2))
 (segment (start 98.416628 24.501) (end 96.811 24.501) (width 0.3) (layer "F.Cu") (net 8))
 (segment (start 99 41.195) (end 99 39.5) (width 0.3) (layer "F.Cu") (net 8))
 (segment (start 105.025 47.22) (end 99 41.195) (width 0.3) (layer "F.Cu") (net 8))
 (segment (start 99.501 29.999) (end 99.501 25.585372) (width 0.3) (layer "F.Cu") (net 8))
 (segment (start 98.5 31) (end 99.501 29.999) (width 0.3) (layer "F.Cu") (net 8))
 (segment (start 96.811 24.501) (end 96.06 23.75) (width 0.3) (layer "F.Cu") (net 8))
 (segment (start 107.175 47.22) (end 106.1 47.22) (width 0.3) (layer "F.Cu") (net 8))
 (segment (start 99.501 25.585372) (end 98.416628 24.501) (width 0.3) (layer "F.Cu") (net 8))
 (segment (start 106.1 47.22) (end 105.025 47.22) (width 0.3) (layer "F.Cu") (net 8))
 (via (at 99 39.5) (size 0.6) (drill 0.3) (layers "F.Cu" "B.Cu") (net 8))
 (segment (start 97.499 32.249) (end 97.499 25.189) (width 0.3) (layer "B.Cu") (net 8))
 (segment (start 97.499 25.189) (end 96.06 23.75) (width 0.3) (layer "B.Cu") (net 8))
 (segment (start 98.5 33.25) (end 98.5 31) (width 0.3) (layer "B.Cu") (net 8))
 (segment (start 99 39.5) (end 98.5 39) (width 0.3) (layer "B.Cu") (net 8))
 (segment (start 98.5 39) (end 98.5 33.25) (width 0.3) (layer "B.Cu") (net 8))
 (segment (start 98.5 33.25) (end 97.499 32.249) (width 0.3) (layer "B.Cu") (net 8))
 (segment (start 96.12 30.464917) (end 98.106083 32.451) (width 0.3) (layer "F.Cu") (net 9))
 (segment (start 107.049 32.451) (end 108.5 31) (width 0.3) (layer "F.Cu") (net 9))
 (segment (start 106.1 44.68) (end 96.12 34.7) (width 0.3) (layer "F.Cu") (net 9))
 (segment (start 108.5 31) (end 108.5 33) (width 0.3) (layer "F.Cu") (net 9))
 (segment (start 98.106083 32.451) (end 107.049 32.451) (width 0.3) (layer "F.Cu") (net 9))
 (segment (start 96.12 27) (end 96.12 30.464917) (width 0.3) (layer "F.Cu") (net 9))
 (segment (start 103 36.829347) (end 103 40.25) (width 0.3) (layer "F.Cu") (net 9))
 (segment (start 103 40.25) (end 106.1 43.35) (width 0.3) (layer "F.Cu") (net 9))
 (segment (start 106.329347 33.5) (end 103 36.829347) (width 0.3) (layer "F.Cu") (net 9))
 (segment (start 96.12 34.7) (end 96.12 27) (width 0.3) (layer "F.Cu") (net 9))
 (segment (start 108 33.5) (end 106.329347 33.5) (width 0.3) (layer "F.Cu") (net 9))
 (segment (start 108.5 33) (end 108 33.5) (width 0.3) (layer "F.Cu") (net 9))
 (segment (start 106.1 43.35) (end 106.1 44.68) (width 0.3) (layer "F.Cu") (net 9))
 (segment (start 107.175 57.38) (end 106.1 57.38) (width 0.3) (layer "F.Cu") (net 4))
 (segment (start 107.175 59.92) (end 106.1 59.92) (width 0.3) (layer "F.Cu") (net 3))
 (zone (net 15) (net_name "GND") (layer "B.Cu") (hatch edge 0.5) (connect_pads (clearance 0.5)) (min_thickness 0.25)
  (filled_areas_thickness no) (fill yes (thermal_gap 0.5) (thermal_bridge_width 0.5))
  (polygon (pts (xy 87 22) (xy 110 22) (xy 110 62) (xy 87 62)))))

